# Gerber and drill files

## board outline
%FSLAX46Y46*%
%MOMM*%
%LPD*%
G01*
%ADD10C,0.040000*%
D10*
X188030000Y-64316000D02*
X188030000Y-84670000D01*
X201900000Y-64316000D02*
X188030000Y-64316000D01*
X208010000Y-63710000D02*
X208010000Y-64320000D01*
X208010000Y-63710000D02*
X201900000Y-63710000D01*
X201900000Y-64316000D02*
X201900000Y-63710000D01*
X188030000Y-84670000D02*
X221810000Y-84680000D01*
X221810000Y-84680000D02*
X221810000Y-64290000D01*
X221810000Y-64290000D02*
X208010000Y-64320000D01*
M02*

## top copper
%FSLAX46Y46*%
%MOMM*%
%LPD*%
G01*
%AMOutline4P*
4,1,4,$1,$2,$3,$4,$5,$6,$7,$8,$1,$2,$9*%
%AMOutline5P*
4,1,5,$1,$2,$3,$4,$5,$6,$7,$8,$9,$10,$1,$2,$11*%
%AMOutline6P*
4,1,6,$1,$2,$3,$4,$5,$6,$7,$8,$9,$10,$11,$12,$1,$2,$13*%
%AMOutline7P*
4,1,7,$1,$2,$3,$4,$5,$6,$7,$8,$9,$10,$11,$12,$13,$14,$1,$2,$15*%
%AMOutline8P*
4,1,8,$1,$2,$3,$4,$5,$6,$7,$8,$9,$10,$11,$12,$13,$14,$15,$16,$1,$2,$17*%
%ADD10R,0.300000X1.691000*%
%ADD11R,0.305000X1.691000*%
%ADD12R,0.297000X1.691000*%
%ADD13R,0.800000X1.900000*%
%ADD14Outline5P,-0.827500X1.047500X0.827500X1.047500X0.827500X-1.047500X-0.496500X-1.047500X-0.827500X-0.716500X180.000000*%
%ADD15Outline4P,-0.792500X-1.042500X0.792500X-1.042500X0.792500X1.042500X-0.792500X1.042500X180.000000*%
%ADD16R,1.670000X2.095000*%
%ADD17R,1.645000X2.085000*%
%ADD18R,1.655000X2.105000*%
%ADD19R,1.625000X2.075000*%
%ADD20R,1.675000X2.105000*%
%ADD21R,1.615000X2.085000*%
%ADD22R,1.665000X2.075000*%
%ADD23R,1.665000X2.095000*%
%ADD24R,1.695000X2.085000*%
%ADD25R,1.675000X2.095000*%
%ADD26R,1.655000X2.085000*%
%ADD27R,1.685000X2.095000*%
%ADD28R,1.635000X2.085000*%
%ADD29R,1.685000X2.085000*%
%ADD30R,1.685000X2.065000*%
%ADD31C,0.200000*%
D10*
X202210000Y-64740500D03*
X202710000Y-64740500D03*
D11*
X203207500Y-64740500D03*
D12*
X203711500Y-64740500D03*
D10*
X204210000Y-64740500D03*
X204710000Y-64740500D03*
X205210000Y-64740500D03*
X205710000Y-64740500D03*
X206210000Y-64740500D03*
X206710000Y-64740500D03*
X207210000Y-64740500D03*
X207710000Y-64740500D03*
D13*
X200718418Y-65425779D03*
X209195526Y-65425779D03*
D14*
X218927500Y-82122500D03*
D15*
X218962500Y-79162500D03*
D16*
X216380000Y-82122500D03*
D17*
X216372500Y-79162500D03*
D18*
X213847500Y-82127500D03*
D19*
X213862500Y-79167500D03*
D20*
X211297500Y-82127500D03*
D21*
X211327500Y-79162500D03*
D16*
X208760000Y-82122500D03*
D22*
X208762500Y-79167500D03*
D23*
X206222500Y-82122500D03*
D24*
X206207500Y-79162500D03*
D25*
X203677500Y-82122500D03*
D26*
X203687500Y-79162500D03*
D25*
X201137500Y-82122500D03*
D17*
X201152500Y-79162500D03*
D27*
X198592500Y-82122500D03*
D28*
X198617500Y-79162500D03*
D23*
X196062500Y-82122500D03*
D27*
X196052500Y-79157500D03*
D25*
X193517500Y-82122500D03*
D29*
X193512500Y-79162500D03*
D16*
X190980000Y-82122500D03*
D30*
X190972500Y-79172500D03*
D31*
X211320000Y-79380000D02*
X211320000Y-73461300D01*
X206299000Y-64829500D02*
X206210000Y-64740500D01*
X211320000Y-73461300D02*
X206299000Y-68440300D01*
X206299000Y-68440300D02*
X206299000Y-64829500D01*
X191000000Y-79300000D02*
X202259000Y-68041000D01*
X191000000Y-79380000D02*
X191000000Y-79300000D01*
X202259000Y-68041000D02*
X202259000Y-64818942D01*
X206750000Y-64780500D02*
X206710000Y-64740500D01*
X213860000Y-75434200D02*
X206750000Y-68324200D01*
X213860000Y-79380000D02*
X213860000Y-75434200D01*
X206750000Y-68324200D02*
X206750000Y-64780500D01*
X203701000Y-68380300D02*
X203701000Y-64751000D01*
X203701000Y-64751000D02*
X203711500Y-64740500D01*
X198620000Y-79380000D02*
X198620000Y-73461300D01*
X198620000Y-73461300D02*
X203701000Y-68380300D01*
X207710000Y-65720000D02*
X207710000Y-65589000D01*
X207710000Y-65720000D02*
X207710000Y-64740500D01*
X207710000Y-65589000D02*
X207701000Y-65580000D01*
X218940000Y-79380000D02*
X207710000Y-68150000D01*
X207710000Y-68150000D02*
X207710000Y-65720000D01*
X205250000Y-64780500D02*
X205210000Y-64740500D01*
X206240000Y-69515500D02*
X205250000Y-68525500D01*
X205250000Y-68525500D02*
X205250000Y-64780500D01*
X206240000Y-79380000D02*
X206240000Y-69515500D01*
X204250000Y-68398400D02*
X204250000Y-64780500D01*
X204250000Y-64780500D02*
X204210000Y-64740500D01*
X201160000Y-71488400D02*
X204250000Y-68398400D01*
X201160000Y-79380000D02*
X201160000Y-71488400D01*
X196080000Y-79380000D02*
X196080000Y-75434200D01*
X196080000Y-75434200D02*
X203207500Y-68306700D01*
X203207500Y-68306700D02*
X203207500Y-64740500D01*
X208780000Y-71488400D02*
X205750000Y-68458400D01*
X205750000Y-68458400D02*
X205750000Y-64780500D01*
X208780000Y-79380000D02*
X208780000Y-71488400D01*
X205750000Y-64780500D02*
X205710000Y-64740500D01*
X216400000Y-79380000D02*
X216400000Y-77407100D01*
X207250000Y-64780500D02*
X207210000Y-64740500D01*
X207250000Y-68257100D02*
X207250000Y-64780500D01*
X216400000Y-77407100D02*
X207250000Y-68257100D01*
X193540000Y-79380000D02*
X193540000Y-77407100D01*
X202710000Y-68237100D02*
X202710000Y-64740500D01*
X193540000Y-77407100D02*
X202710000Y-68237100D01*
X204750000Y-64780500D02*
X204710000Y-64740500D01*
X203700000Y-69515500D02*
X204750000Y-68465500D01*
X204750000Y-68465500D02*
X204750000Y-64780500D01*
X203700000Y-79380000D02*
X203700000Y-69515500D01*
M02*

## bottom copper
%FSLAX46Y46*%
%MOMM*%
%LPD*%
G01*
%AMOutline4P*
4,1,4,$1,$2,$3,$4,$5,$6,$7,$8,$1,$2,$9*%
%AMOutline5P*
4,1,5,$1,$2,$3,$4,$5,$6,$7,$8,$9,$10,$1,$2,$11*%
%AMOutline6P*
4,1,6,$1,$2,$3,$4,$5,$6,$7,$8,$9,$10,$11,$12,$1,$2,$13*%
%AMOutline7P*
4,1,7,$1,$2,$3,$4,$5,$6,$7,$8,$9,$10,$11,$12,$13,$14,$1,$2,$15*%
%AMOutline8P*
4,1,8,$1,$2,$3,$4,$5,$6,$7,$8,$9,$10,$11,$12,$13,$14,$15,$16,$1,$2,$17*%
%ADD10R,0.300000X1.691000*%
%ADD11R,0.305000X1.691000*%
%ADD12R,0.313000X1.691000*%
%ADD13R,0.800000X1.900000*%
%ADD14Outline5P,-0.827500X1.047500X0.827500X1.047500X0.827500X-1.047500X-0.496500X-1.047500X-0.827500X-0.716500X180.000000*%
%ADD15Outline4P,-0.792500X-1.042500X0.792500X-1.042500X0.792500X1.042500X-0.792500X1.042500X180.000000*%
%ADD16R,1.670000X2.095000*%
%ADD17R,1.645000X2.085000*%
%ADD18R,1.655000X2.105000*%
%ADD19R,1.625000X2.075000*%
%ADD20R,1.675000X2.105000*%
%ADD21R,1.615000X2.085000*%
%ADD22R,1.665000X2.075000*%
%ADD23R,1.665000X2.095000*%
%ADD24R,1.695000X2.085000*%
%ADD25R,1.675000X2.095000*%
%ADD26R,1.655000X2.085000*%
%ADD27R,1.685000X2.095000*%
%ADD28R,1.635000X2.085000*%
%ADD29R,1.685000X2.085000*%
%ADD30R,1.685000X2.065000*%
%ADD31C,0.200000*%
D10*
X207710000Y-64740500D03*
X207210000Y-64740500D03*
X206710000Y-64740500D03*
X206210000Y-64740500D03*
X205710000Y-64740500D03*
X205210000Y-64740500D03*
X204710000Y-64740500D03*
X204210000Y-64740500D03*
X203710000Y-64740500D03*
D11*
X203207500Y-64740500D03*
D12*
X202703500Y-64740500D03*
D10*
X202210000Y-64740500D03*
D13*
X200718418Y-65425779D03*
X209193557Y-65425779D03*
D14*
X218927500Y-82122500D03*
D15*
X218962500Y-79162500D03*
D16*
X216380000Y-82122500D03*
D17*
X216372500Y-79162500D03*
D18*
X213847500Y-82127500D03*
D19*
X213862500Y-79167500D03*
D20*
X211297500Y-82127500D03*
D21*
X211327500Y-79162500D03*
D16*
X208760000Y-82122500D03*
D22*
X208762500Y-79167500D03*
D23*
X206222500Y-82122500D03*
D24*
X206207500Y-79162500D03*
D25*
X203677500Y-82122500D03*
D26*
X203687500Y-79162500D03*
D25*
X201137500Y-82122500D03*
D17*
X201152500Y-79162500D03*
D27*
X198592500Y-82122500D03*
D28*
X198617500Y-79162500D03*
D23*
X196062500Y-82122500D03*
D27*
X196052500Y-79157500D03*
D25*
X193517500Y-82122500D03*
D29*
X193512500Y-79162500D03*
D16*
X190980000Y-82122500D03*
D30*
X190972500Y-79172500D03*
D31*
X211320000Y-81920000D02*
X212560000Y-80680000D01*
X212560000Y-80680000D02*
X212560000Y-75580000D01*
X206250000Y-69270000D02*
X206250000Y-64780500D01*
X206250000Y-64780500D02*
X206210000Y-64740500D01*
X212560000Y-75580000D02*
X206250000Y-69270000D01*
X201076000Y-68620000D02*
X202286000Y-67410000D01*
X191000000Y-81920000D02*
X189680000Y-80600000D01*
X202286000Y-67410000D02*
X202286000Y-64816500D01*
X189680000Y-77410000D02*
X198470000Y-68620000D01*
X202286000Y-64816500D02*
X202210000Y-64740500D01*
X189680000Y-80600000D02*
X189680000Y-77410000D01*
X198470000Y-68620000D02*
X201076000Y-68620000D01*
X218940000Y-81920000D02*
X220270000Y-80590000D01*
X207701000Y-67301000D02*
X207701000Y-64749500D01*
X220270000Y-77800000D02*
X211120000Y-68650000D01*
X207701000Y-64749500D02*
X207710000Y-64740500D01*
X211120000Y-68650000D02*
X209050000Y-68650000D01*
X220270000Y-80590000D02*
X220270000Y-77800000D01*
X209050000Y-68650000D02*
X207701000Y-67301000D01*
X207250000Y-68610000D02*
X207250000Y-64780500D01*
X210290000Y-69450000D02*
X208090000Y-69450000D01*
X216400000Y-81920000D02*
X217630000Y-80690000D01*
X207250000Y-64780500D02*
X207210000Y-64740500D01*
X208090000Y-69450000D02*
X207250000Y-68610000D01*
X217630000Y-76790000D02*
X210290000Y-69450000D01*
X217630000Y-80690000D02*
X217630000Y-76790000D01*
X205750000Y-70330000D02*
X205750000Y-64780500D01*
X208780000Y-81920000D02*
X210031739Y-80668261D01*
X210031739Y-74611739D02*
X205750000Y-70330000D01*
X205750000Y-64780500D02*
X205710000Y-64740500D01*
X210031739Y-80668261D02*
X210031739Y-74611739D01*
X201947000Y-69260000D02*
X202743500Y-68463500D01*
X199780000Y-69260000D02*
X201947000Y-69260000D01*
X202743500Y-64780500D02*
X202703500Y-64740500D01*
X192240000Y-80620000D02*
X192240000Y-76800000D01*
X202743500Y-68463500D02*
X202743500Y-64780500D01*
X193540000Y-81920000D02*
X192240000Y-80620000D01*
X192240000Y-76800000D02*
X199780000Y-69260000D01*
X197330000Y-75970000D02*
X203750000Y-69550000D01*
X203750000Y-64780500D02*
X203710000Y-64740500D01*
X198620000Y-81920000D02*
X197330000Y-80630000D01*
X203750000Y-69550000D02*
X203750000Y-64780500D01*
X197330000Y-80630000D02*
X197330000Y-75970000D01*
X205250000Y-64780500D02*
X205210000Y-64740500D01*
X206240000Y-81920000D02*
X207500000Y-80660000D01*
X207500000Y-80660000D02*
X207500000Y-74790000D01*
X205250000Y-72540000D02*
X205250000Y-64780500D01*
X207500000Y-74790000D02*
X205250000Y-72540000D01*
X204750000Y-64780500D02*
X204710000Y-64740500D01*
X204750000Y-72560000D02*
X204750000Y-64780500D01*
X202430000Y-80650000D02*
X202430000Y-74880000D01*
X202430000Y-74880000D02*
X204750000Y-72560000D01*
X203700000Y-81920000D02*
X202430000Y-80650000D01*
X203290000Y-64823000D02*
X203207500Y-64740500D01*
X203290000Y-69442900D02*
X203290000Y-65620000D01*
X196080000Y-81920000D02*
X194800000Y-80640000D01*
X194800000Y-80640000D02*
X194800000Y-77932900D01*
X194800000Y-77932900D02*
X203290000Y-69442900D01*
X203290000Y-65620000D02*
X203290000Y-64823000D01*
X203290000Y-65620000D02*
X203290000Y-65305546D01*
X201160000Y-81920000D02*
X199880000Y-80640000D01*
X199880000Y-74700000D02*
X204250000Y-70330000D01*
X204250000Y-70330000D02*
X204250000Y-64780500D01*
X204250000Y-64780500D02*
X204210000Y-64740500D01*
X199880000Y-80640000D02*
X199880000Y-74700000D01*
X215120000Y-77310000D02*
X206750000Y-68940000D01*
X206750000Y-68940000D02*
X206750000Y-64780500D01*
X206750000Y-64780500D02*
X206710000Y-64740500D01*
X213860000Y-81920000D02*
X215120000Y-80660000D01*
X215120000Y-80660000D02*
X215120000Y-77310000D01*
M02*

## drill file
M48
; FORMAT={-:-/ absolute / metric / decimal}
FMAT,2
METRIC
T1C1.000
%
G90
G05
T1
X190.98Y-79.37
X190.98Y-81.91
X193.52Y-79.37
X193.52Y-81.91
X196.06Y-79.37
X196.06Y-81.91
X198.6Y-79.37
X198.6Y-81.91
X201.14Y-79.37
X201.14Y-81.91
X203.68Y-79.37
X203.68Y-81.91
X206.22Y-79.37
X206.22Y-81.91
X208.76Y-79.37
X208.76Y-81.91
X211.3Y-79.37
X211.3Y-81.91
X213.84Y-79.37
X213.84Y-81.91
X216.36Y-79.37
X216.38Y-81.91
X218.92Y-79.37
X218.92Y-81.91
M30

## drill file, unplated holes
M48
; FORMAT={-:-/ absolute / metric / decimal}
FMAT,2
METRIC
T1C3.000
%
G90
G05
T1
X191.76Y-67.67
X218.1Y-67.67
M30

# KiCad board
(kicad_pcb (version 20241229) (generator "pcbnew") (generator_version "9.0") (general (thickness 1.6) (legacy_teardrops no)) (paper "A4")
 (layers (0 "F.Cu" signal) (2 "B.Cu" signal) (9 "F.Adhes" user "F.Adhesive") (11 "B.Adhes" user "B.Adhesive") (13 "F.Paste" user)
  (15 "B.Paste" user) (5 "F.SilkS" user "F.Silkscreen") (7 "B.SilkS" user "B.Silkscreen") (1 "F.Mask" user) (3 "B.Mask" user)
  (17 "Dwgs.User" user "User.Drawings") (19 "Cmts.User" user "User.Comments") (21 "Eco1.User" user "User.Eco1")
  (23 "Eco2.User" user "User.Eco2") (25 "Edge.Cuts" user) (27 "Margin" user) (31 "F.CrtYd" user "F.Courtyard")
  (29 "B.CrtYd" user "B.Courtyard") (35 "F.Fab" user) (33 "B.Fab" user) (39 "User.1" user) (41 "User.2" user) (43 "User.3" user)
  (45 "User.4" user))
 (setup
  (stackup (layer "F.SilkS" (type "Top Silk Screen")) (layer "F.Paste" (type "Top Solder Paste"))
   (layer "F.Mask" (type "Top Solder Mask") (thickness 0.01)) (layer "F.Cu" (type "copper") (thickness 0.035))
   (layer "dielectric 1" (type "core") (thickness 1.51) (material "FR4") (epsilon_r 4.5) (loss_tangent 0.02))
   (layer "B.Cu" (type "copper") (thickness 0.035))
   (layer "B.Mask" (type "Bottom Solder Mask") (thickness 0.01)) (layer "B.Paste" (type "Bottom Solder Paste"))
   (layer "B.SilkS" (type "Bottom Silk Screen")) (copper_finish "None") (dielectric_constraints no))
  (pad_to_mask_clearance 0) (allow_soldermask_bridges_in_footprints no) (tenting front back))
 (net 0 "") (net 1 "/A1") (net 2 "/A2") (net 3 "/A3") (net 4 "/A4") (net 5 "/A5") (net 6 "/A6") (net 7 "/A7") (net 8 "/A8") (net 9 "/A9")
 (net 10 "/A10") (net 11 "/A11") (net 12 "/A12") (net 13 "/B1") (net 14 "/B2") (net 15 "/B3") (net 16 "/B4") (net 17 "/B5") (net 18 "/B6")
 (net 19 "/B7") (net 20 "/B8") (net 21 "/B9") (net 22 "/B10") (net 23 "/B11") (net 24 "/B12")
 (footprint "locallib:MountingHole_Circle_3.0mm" (layer "F.Cu") (at 218.1 67.67)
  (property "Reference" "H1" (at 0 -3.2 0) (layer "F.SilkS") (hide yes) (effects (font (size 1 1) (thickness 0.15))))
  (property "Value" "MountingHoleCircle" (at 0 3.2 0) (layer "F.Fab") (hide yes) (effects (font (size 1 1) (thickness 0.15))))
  (pad "" np_thru_hole circle (at 0 0) (size 3 3) (drill 3) (layers "*.Cu" "*.Mask")))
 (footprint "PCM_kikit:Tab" (layer "F.Cu") (at 216.02 84.84 90)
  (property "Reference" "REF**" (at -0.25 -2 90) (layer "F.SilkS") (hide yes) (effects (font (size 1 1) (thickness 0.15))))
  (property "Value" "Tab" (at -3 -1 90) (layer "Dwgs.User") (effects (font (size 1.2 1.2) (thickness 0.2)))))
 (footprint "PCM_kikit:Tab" (layer "F.Cu") (at 216 64.13 -90)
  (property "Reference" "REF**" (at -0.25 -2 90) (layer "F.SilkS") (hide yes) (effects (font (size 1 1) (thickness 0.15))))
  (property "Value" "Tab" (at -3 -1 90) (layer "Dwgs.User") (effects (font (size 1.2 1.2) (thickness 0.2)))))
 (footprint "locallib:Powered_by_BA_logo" (layer "F.Cu") (at 193.79 72.61)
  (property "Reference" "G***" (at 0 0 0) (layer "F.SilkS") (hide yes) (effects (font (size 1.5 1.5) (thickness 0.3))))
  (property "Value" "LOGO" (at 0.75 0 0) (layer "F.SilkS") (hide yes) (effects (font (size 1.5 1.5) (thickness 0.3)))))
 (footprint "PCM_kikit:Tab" (layer "F.Cu") (at 187.87 82.95)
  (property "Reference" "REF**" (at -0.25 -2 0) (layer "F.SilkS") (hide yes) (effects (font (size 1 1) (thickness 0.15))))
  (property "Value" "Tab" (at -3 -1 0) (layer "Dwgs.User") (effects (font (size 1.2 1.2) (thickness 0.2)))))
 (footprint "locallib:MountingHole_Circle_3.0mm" (layer "F.Cu") (at 191.76 67.67)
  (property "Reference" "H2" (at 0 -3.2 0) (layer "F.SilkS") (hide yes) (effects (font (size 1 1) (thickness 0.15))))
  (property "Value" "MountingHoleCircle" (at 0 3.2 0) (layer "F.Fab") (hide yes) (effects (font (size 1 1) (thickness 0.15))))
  (pad "" np_thru_hole circle (at 0 0) (size 3 3) (drill 3) (layers "*.Cu" "*.Mask")))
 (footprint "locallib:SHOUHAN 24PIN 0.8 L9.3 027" (layer "F.Cu") (at 204.96 64.57 180)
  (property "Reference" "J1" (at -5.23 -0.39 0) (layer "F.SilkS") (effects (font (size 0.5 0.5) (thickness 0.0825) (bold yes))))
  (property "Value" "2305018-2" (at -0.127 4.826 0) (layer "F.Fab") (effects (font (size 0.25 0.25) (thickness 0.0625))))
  (pad "A1" smd rect (at 2.75 -0.1705 180) (size 0.3 1.691) (layers "F.Cu" "F.Mask" "F.Paste") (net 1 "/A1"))
  (pad "A2" smd rect (at 2.25 -0.1705 180) (size 0.3 1.691) (layers "F.Cu" "F.Mask" "F.Paste") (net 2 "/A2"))
  (pad "A3" smd rect (at 1.7525 -0.1705 180) (size 0.305 1.691) (layers "F.Cu" "F.Mask" "F.Paste") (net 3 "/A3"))
  (pad "A4" smd rect (at 1.2485 -0.1705 180) (size 0.297 1.691) (layers "F.Cu" "F.Mask" "F.Paste") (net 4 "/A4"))
  (pad "A5" smd rect (at 0.75 -0.1705 180) (size 0.3 1.691) (layers "F.Cu" "F.Mask" "F.Paste") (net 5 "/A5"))
  (pad "A6" smd rect (at 0.25 -0.1705 180) (size 0.3 1.691) (layers "F.Cu" "F.Mask" "F.Paste") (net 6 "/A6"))
  (pad "A7" smd rect (at -0.25 -0.1705 180) (size 0.3 1.691) (layers "F.Cu" "F.Mask" "F.Paste") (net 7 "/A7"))
  (pad "A8" smd rect (at -0.75 -0.1705 180) (size 0.3 1.691) (layers "F.Cu" "F.Mask" "F.Paste") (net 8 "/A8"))
  (pad "A9" smd rect (at -1.25 -0.1705 180) (size 0.3 1.691) (layers "F.Cu" "F.Mask" "F.Paste") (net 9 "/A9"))
  (pad "A10" smd rect (at -1.75 -0.1705 180) (size 0.3 1.691) (layers "F.Cu" "F.Mask" "F.Paste") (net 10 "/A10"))
  (pad "A11" smd rect (at -2.25 -0.1705 180) (size 0.3 1.691) (layers "F.Cu" "F.Mask" "F.Paste") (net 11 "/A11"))
  (pad "A12" smd rect (at -2.75 -0.1705 180) (size 0.3 1.691) (layers "F.Cu" "F.Mask" "F.Paste") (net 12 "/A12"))
  (pad "B1" smd rect (at -2.75 -0.1705 180) (size 0.3 1.691) (layers "B.Cu" "B.Mask" "B.Paste") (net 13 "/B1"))
  (pad "B2" smd rect (at -2.25 -0.1705 180) (size 0.3 1.691) (layers "B.Cu" "B.Mask" "B.Paste") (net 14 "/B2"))
  (pad "B3" smd rect (at -1.75 -0.1705 180) (size 0.3 1.691) (layers "B.Cu" "B.Mask" "B.Paste") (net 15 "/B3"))
  (pad "B4" smd rect (at -1.25 -0.1705 180) (size 0.3 1.691) (layers "B.Cu" "B.Mask" "B.Paste") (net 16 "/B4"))
  (pad "B5" smd rect (at -0.75 -0.1705 180) (size 0.3 1.691) (layers "B.Cu" "B.Mask" "B.Paste") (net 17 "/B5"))
  (pad "B6" smd rect (at -0.25 -0.1705 180) (size 0.3 1.691) (layers "B.Cu" "B.Mask" "B.Paste") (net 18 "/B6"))
  (pad "B7" smd rect (at 0.25 -0.1705 180) (size 0.3 1.691) (layers "B.Cu" "B.Mask" "B.Paste") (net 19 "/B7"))
  (pad "B8" smd rect (at 0.75 -0.1705 180) (size 0.3 1.691) (layers "B.Cu" "B.Mask" "B.Paste") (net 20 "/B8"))
  (pad "B9" smd rect (at 1.25 -0.1705 180) (size 0.3 1.691) (layers "B.Cu" "B.Mask" "B.Paste") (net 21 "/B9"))
  (pad "B10" smd rect (at 1.7525 -0.1705 180) (size 0.305 1.691) (layers "B.Cu" "B.Mask" "B.Paste") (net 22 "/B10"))
  (pad "B11" smd rect (at 2.2565 -0.1705 180) (size 0.313 1.691) (layers "B.Cu" "B.Mask" "B.Paste") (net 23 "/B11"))
  (pad "B12" smd rect (at 2.75 -0.1705 180) (size 0.3 1.691) (layers "B.Cu" "B.Mask" "B.Paste") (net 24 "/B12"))
  (pad "S1" smd rect (at 4.241582 -0.855779 180) (size 0.8 1.9) (layers "F.Cu" "F.Mask" "F.Paste"))
  (pad "S2" smd rect (at -4.235526 -0.855779 180) (size 0.8 1.9) (layers "F.Cu" "F.Mask" "F.Paste"))
  (pad "S3" smd rect (at 4.241582 -0.855779 180) (size 0.8 1.9) (layers "B.Cu" "B.Mask" "B.Paste"))
  (pad "S4" smd rect (at -4.233557 -0.855779 180) (size 0.8 1.9) (layers "B.Cu" "B.Mask" "B.Paste")))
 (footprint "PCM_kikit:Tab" (layer "F.Cu") (at 221.99 83.06 180)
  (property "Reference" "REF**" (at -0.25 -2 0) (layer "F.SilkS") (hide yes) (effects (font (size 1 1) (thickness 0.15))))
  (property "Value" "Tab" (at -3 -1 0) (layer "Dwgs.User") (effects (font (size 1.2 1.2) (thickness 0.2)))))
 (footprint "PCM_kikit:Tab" (layer "F.Cu") (at 194.02 84.82 90)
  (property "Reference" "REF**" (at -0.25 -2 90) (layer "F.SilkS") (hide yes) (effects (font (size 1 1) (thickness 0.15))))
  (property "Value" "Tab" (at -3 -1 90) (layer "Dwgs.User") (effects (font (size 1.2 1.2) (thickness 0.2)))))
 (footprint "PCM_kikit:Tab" (layer "F.Cu") (at 221.96 66.09 180)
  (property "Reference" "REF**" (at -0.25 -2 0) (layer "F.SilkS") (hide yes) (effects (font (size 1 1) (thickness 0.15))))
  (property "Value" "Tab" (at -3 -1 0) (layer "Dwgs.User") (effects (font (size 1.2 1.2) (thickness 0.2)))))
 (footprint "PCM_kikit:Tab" (layer "F.Cu") (at 193.95 64.14 -90)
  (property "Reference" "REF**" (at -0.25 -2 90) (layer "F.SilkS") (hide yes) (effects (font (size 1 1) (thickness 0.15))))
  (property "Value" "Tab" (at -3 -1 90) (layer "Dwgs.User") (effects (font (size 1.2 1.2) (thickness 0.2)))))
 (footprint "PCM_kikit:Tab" (layer "F.Cu") (at 187.87 66.09)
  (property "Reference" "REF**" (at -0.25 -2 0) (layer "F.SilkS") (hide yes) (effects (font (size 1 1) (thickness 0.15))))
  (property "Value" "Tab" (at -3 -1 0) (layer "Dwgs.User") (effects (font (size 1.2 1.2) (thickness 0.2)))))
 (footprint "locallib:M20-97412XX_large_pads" (layer "B.Cu") (at 218.92 81.91 180)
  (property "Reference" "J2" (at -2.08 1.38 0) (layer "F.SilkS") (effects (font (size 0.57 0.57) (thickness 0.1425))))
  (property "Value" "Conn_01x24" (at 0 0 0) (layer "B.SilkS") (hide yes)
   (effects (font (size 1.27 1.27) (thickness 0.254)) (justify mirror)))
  (pad "1" thru_hole roundrect (at 0 0 180) (size 1.655 2.095) (drill 1 (offset -0.0075 -0.2125)) (layers "*.Cu" "*.Mask")
   (remove_unused_layers no) (roundrect_rratio 0) (chamfer_ratio 0.2) (chamfer bottom_left) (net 13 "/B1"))
  (pad "2" thru_hole trapezoid (at 0 2.54 180) (size 1.585 2.085) (drill 1 (offset -0.0425 0.2075)) (layers "*.Cu" "*.Mask")
   (remove_unused_layers no) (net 12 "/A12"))
  (pad "3" thru_hole rect (at 2.54 0 180) (size 1.67 2.095) (drill 1 (offset 0 -0.2125)) (layers "*.Cu" "*.Mask") (remove_unused_layers no)
   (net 14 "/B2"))
  (pad "4" thru_hole rect (at 2.56 2.54 180) (size 1.645 2.085) (drill 1 (offset -0.0125 0.2075)) (layers "*.Cu" "*.Mask")
   (remove_unused_layers no) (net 11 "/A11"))
  (pad "5" thru_hole rect (at 5.08 0 180) (size 1.655 2.105) (drill 1 (offset -0.0075 -0.2175)) (layers "*.Cu" "*.Mask")
   (remove_unused_layers no) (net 15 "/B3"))
  (pad "6" thru_hole rect (at 5.08 2.54 180) (size 1.625 2.075) (drill 1 (offset -0.0225 0.2025)) (layers "*.Cu" "*.Mask")
   (remove_unused_layers no) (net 10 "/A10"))
  (pad "7" thru_hole rect (at 7.62 0 180) (size 1.675 2.105) (drill 1 (offset 0.0025 -0.2175)) (layers "*.Cu" "*.Mask")
   (remove_unused_layers no) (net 16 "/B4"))
  (pad "8" thru_hole rect (at 7.62 2.54 180) (size 1.615 2.085) (drill 1 (offset -0.0275 0.2075)) (layers "*.Cu" "*.Mask")
   (remove_unused_layers no) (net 9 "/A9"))
  (pad "9" thru_hole rect (at 10.16 0 180) (size 1.67 2.095) (drill 1 (offset 0 -0.2125)) (layers "*.Cu" "*.Mask") (remove_unused_layers no)
   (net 17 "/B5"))
  (pad "10" thru_hole rect (at 10.16 2.54 180) (size 1.665 2.075) (drill 1 (offset -0.0025 0.2025)) (layers "*.Cu" "*.Mask")
   (remove_unused_layers no) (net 8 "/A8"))
  (pad "11" thru_hole rect (at 12.7 0 180) (size 1.665 2.095) (drill 1 (offset -0.0025 -0.2125)) (layers "*.Cu" "*.Mask")
   (remove_unused_layers no) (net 18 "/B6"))
  (pad "12" thru_hole rect (at 12.7 2.54 180) (size 1.695 2.085) (drill 1 (offset 0.0125 0.2075)) (layers "*.Cu" "*.Mask")
   (remove_unused_layers no) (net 7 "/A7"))
  (pad "13" thru_hole rect (at 15.24 0 180) (size 1.675 2.095) (drill 1 (offset 0.0025 -0.2125)) (layers "*.Cu" "*.Mask")
   (remove_unused_layers no) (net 19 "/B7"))
  (pad "14" thru_hole rect (at 15.24 2.54 180) (size 1.655 2.085) (drill 1 (offset -0.0075 0.2075)) (layers "*.Cu" "*.Mask")
   (remove_unused_layers no) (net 6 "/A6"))
  (pad "15" thru_hole rect (at 17.78 0 180) (size 1.675 2.095) (drill 1 (offset 0.0025 -0.2125)) (layers "*.Cu" "*.Mask")
   (remove_unused_layers no) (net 20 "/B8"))
  (pad "16" thru_hole rect (at 17.78 2.54 180) (size 1.645 2.085) (drill 1 (offset -0.0125 0.2075)) (layers "*.Cu" "*.Mask")
   (remove_unused_layers no) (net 5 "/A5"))
  (pad "17" thru_hole rect (at 20.32 0 180) (size 1.685 2.095) (drill 1 (offset 0.0075 -0.2125)) (layers "*.Cu" "*.Mask")
   (remove_unused_layers no) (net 21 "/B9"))
  (pad "18" thru_hole rect (at 20.32 2.54 180) (size 1.635 2.085) (drill 1 (offset -0.0175 0.2075)) (layers "*.Cu" "*.Mask")
   (remove_unused_layers no) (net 4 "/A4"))
  (pad "19" thru_hole rect (at 22.86 0 180) (size 1.665 2.095) (drill 1 (offset -0.0025 -0.2125)) (layers "*.Cu" "*.Mask")
   (remove_unused_layers no) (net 22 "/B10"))
  (pad "20" thru_hole rect (at 22.86 2.54 180) (size 1.685 2.095) (drill 1 (offset 0.0075 0.2125)) (layers "*.Cu" "*.Mask")
   (remove_unused_layers no) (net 3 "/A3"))
  (pad "21" thru_hole rect (at 25.4 0 180) (size 1.675 2.095) (drill 1 (offset 0.0025 -0.2125)) (layers "*.Cu" "*.Mask")
   (remove_unused_layers no) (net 23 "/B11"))
  (pad "22" thru_hole rect (at 25.4 2.54 180) (size 1.685 2.085) (drill 1 (offset 0.0075 0.2075)) (layers "*.Cu" "*.Mask")
   (remove_unused_layers no) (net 2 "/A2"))
  (pad "23" thru_hole rect (at 27.94 0 180) (size 1.67 2.095) (drill 1 (offset 0 -0.2125)) (layers "*.Cu" "*.Mask")
   (remove_unused_layers no) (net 24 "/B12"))
  (pad "24" thru_hole rect (at 27.94 2.54 180) (size 1.685 2.065) (drill 1 (offset 0.0075 0.1975)) (layers "*.Cu" "*.Mask")
   (remove_unused_layers no) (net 1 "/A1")))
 (gr_line (start 188.03 64.316) (end 188.03 84.67) (stroke (width 0.04) (type solid)) (layer "Edge.Cuts"))
 (gr_line (start 201.9 64.316) (end 188.03 64.316) (stroke (width 0.04) (type solid)) (layer "Edge.Cuts"))
 (gr_line (start 208.01 63.71) (end 208.01 64.32) (stroke (width 0.04) (type solid)) (layer "Edge.Cuts"))
 (gr_line (start 208.01 63.71) (end 201.9 63.71) (stroke (width 0.04) (type solid)) (layer "Edge.Cuts"))
 (gr_line (start 201.9 64.316) (end 201.9 63.71) (stroke (width 0.04) (type solid)) (layer "Edge.Cuts"))
 (gr_line (start 188.03 84.67) (end 221.81 84.68) (stroke (width 0.04) (type solid)) (layer "Edge.Cuts"))
 (gr_line (start 221.81 84.68) (end 221.81 64.29) (stroke (width 0.04) (type solid)) (layer "Edge.Cuts"))
 (gr_line (start 221.81 64.29) (end 208.01 64.32) (stroke (width 0.04) (type solid)) (layer "Edge.Cuts"))
 (segment (start 211.32 81.92) (end 212.56 80.68) (width 0.2) (layer "B.Cu") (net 16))
 (segment (start 212.56 80.68) (end 212.56 75.58) (width 0.2) (layer "B.Cu") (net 16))
 (segment (start 206.25 69.27) (end 206.25 64.7805) (width 0.2) (layer "B.Cu") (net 16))
 (segment (start 206.25 64.7805) (end 206.21 64.7405) (width 0.2) (layer "B.Cu") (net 16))
 (segment (start 212.56 75.58) (end 206.25 69.27) (width 0.2) (layer "B.Cu") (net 16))
 (segment (start 201.076 68.62) (end 202.286 67.41) (width 0.2) (layer "B.Cu") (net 24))
 (segment (start 191 81.92) (end 189.68 80.6) (width 0.2) (layer "B.Cu") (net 24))
 (segment (start 202.286 67.41) (end 202.286 64.8165) (width 0.2) (layer "B.Cu") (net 24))
 (segment (start 189.68 77.41) (end 198.47 68.62) (width 0.2) (layer "B.Cu") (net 24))
 (segment (start 202.286 64.8165) (end 202.21 64.7405) (width 0.2) (layer "B.Cu") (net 24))
 (segment (start 189.68 80.6) (end 189.68 77.41) (width 0.2) (layer "B.Cu") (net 24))
 (segment (start 198.47 68.62) (end 201.076 68.62) (width 0.2) (layer "B.Cu") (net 24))
 (segment (start 218.94 81.92) (end 220.27 80.59) (width 0.2) (layer "B.Cu") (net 13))
 (segment (start 207.701 67.301) (end 207.701 64.7495) (width 0.2) (layer "B.Cu") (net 13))
 (segment (start 220.27 77.8) (end 211.12 68.65) (width 0.2) (layer "B.Cu") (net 13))
 (segment (start 207.701 64.7495) (end 207.71 64.7405) (width 0.2) (layer "B.Cu") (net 13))
 (segment (start 211.12 68.65) (end 209.05 68.65) (width 0.2) (layer "B.Cu") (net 13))
 (segment (start 220.27 80.59) (end 220.27 77.8) (width 0.2) (layer "B.Cu") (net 13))
 (segment (start 209.05 68.65) (end 207.701 67.301) (width 0.2) (layer "B.Cu") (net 13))
 (segment (start 207.25 68.61) (end 207.25 64.7805) (width 0.2) (layer "B.Cu") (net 14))
 (segment (start 210.29 69.45) (end 208.09 69.45) (width 0.2) (layer "B.Cu") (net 14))
 (segment (start 216.4 81.92) (end 217.63 80.69) (width 0.2) (layer "B.Cu") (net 14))
 (segment (start 207.25 64.7805) (end 207.21 64.7405) (width 0.2) (layer "B.Cu") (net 14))
 (segment (start 208.09 69.45) (end 207.25 68.61) (width 0.2) (layer "B.Cu") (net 14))
 (segment (start 217.63 76.79) (end 210.29 69.45) (width 0.2) (layer "B.Cu") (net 14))
 (segment (start 217.63 80.69) (end 217.63 76.79) (width 0.2) (layer "B.Cu") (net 14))
 (segment (start 211.32 79.38) (end 211.32 73.4613) (width 0.2) (layer "F.Cu") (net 9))
 (segment (start 206.299 64.8295) (end 206.21 64.7405) (width 0.2) (layer "F.Cu") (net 9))
 (segment (start 211.32 73.4613) (end 206.299 68.4403) (width 0.2) (layer "F.Cu") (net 9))
 (segment (start 206.299 68.4403) (end 206.299 64.8295) (width 0.2) (layer "F.Cu") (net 9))
 (segment (start 205.75 70.33) (end 205.75 64.7805) (width 0.2) (layer "B.Cu") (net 17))
 (segment (start 208.78 81.92) (end 210.031739 80.668261) (width 0.2) (layer "B.Cu") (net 17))
 (segment (start 210.031739 74.611739) (end 205.75 70.33) (width 0.2) (layer "B.Cu") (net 17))
 (segment (start 205.75 64.7805) (end 205.71 64.7405) (width 0.2) (layer "B.Cu") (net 17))
 (segment (start 210.031739 80.668261) (end 210.031739 74.611739) (width 0.2) (layer "B.Cu") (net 17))
 (segment (start 201.947 69.26) (end 202.7435 68.4635) (width 0.2) (layer "B.Cu") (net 23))
 (segment (start 199.78 69.26) (end 201.947 69.26) (width 0.2) (layer "B.Cu") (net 23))
 (segment (start 202.7435 64.7805) (end 202.7035 64.7405) (width 0.2) (layer "B.Cu") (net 23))
 (segment (start 192.24 80.62) (end 192.24 76.8) (width 0.2) (layer "B.Cu") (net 23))
 (segment (start 202.7435 68.4635) (end 202.7435 64.7805) (width 0.2) (layer "B.Cu") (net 23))
 (segment (start 193.54 81.92) (end 192.24 80.62) (width 0.2) (layer "B.Cu") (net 23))
 (segment (start 192.24 76.8) (end 199.78 69.26) (width 0.2) (layer "B.Cu") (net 23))
 (segment (start 197.33 75.97) (end 203.75 69.55) (width 0.2) (layer "B.Cu") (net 21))
 (segment (start 203.75 64.7805) (end 203.71 64.7405) (width 0.2) (layer "B.Cu") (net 21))
 (segment (start 198.62 81.92) (end 197.33 80.63) (width 0.2) (layer "B.Cu") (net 21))
 (segment (start 203.75 69.55) (end 203.75 64.7805) (width 0.2) (layer "B.Cu") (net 21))
 (segment (start 197.33 80.63) (end 197.33 75.97) (width 0.2) (layer "B.Cu") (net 21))
 (segment (start 205.25 64.7805) (end 205.21 64.7405) (width 0.2) (layer "B.Cu") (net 18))
 (segment (start 206.24 81.92) (end 207.5 80.66) (width 0.2) (layer "B.Cu") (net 18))
 (segment (start 207.5 80.66) (end 207.5 74.79) (width 0.2) (layer "B.Cu") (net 18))
 (segment (start 205.25 72.54) (end 205.25 64.7805) (width 0.2) (layer "B.Cu") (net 18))
 (segment (start 207.5 74.79) (end 205.25 72.54) (width 0.2) (layer "B.Cu") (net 18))
 (segment (start 204.75 64.7805) (end 204.71 64.7405) (width 0.2) (layer "B.Cu") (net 19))
 (segment (start 204.75 72.56) (end 204.75 64.7805) (width 0.2) (layer "B.Cu") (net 19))
 (segment (start 202.43 80.65) (end 202.43 74.88) (width 0.2) (layer "B.Cu") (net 19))
 (segment (start 202.43 74.88) (end 204.75 72.56) (width 0.2) (layer "B.Cu") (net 19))
 (segment (start 203.7 81.92) (end 202.43 80.65) (width 0.2) (layer "B.Cu") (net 19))
 (segment (start 191 79.3) (end 202.259 68.041) (width 0.2) (layer "F.Cu") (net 1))
 (segment (start 191 79.38) (end 191 79.3) (width 0.2) (layer "F.Cu") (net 1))
 (segment (start 202.259 68.041) (end 202.259 64.818942) (width 0.2) (layer "F.Cu") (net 1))
 (segment (start 203.29 64.823) (end 203.2075 64.7405) (width 0.2) (layer "B.Cu") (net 22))
 (segment (start 203.29 69.4429) (end 203.29 65.62) (width 0.2) (layer "B.Cu") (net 22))
 (segment (start 196.08 81.92) (end 194.8 80.64) (width 0.2) (layer "B.Cu") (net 22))
 (segment (start 194.8 80.64) (end 194.8 77.9329) (width 0.2) (layer "B.Cu") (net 22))
 (segment (start 194.8 77.9329) (end 203.29 69.4429) (width 0.2) (layer "B.Cu") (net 22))
 (segment (start 203.29 65.62) (end 203.29 64.823) (width 0.2) (layer "B.Cu") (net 22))
 (segment (start 203.29 65.62) (end 203.29 65.305546) (width 0.2) (layer "B.Cu") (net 22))
 (segment (start 206.75 64.7805) (end 206.71 64.7405) (width 0.2) (layer "F.Cu") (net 10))
 (segment (start 213.86 75.4342) (end 206.75 68.3242) (width 0.2) (layer "F.Cu") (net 10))
 (segment (start 213.86 79.38) (end 213.86 75.4342) (width 0.2) (layer "F.Cu") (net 10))
 (segment (start 206.75 68.3242) (end 206.75 64.7805) (width 0.2) (layer "F.Cu") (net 10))
 (segment (start 203.701 68.3803) (end 203.701 64.751) (width 0.2) (layer "F.Cu") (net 4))
 (segment (start 203.701 64.751) (end 203.7115 64.7405) (width 0.2) (layer "F.Cu") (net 4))
 (segment (start 198.62 79.38) (end 198.62 73.4613) (width 0.2) (layer "F.Cu") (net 4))
 (segment (start 198.62 73.4613) (end 203.701 68.3803) (width 0.2) (layer "F.Cu") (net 4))
 (segment (start 207.71 65.72) (end 207.71 65.589) (width 0.2) (layer "F.Cu") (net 12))
 (segment (start 207.71 65.72) (end 207.71 64.7405) (width 0.2) (layer "F.Cu") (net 12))
 (segment (start 207.71 65.589) (end 207.701 65.58) (width 0.2) (layer "F.Cu") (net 12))
 (segment (start 218.94 79.38) (end 207.71 68.15) (width 0.2) (layer "F.Cu") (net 12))
 (segment (start 207.71 68.15) (end 207.71 65.72) (width 0.2) (layer "F.Cu") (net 12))
 (segment (start 205.25 64.7805) (end 205.21 64.7405) (width 0.2) (layer "F.Cu") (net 7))
 (segment (start 206.24 69.5155) (end 205.25 68.5255) (width 0.2) (layer "F.Cu") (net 7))
 (segment (start 205.25 68.5255) (end 205.25 64.7805) (width 0.2) (layer "F.Cu") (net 7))
 (segment (start 206.24 79.38) (end 206.24 69.5155) (width 0.2) (layer "F.Cu") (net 7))
 (segment (start 204.25 68.3984) (end 204.25 64.7805) (width 0.2) (layer "F.Cu") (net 5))
 (segment (start 204.25 64.7805) (end 204.21 64.7405) (width 0.2) (layer "F.Cu") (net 5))
 (segment (start 201.16 71.4884) (end 204.25 68.3984) (width 0.2) (layer "F.Cu") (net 5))
 (segment (start 201.16 79.38) (end 201.16 71.4884) (width 0.2) (layer "F.Cu") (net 5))
 (segment (start 196.08 79.38) (end 196.08 75.4342) (width 0.2) (layer "F.Cu") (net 3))
 (segment (start 196.08 75.4342) (end 203.2075 68.3067) (width 0.2) (layer "F.Cu") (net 3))
 (segment (start 203.2075 68.3067) (end 203.2075 64.7405) (width 0.2) (layer "F.Cu") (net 3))
 (segment (start 208.78 71.4884) (end 205.75 68.4584) (width 0.2) (layer "F.Cu") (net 8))
 (segment (start 205.75 68.4584) (end 205.75 64.7805) (width 0.2) (layer "F.Cu") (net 8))
 (segment (start 208.78 79.38) (end 208.78 71.4884) (width 0.2) (layer "F.Cu") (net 8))
 (segment (start 205.75 64.7805) (end 205.71 64.7405) (width 0.2) (layer "F.Cu") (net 8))
 (segment (start 201.16 81.92) (end 199.88 80.64) (width 0.2) (layer "B.Cu") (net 20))
 (segment (start 199.88 74.7) (end 204.25 70.33) (width 0.2) (layer "B.Cu") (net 20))
 (segment (start 204.25 70.33) (end 204.25 64.7805) (width 0.2) (layer "B.Cu") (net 20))
 (segment (start 204.25 64.7805) (end 204.21 64.7405) (width 0.2) (layer "B.Cu") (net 20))
 (segment (start 199.88 80.64) (end 199.88 74.7) (width 0.2) (layer "B.Cu") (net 20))
 (segment (start 216.4 79.38) (end 216.4 77.4071) (width 0.2) (layer "F.Cu") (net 11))
 (segment (start 207.25 64.7805) (end 207.21 64.7405) (width 0.2) (layer "F.Cu") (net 11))
 (segment (start 207.25 68.2571) (end 207.25 64.7805) (width 0.2) (layer "F.Cu") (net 11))
 (segment (start 216.4 77.4071) (end 207.25 68.2571) (width 0.2) (layer "F.Cu") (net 11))
 (segment (start 193.54 79.38) (end 193.54 77.4071) (width 0.2) (layer "F.Cu") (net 2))
 (segment (start 202.71 68.2371) (end 202.71 64.7405) (width 0.2) (layer "F.Cu") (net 2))
 (segment (start 193.54 77.4071) (end 202.71 68.2371) (width 0.2) (layer "F.Cu") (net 2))
 (segment (start 215.12 77.31) (end 206.75 68.94) (width 0.2) (layer "B.Cu") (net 15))
 (segment (start 206.75 68.94) (end 206.75 64.7805) (width 0.2) (layer "B.Cu") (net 15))
 (segment (start 206.75 64.7805) (end 206.71 64.7405) (width 0.2) (layer "B.Cu") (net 15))
 (segment (start 213.86 81.92) (end 215.12 80.66) (width 0.2) (layer "B.Cu") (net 15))
 (segment (start 215.12 80.66) (end 215.12 77.31) (width 0.2) (layer "B.Cu") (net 15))
 (segment (start 204.75 64.7805) (end 204.71 64.7405) (width 0.2) (layer "F.Cu") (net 6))
 (segment (start 203.7 69.5155) (end 204.75 68.4655) (width 0.2) (layer "F.Cu") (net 6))
 (segment (start 204.75 68.4655) (end 204.75 64.7805) (width 0.2) (layer "F.Cu") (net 6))
 (segment (start 203.7 79.38) (end 203.7 69.5155) (width 0.2) (layer "F.Cu") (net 6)))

